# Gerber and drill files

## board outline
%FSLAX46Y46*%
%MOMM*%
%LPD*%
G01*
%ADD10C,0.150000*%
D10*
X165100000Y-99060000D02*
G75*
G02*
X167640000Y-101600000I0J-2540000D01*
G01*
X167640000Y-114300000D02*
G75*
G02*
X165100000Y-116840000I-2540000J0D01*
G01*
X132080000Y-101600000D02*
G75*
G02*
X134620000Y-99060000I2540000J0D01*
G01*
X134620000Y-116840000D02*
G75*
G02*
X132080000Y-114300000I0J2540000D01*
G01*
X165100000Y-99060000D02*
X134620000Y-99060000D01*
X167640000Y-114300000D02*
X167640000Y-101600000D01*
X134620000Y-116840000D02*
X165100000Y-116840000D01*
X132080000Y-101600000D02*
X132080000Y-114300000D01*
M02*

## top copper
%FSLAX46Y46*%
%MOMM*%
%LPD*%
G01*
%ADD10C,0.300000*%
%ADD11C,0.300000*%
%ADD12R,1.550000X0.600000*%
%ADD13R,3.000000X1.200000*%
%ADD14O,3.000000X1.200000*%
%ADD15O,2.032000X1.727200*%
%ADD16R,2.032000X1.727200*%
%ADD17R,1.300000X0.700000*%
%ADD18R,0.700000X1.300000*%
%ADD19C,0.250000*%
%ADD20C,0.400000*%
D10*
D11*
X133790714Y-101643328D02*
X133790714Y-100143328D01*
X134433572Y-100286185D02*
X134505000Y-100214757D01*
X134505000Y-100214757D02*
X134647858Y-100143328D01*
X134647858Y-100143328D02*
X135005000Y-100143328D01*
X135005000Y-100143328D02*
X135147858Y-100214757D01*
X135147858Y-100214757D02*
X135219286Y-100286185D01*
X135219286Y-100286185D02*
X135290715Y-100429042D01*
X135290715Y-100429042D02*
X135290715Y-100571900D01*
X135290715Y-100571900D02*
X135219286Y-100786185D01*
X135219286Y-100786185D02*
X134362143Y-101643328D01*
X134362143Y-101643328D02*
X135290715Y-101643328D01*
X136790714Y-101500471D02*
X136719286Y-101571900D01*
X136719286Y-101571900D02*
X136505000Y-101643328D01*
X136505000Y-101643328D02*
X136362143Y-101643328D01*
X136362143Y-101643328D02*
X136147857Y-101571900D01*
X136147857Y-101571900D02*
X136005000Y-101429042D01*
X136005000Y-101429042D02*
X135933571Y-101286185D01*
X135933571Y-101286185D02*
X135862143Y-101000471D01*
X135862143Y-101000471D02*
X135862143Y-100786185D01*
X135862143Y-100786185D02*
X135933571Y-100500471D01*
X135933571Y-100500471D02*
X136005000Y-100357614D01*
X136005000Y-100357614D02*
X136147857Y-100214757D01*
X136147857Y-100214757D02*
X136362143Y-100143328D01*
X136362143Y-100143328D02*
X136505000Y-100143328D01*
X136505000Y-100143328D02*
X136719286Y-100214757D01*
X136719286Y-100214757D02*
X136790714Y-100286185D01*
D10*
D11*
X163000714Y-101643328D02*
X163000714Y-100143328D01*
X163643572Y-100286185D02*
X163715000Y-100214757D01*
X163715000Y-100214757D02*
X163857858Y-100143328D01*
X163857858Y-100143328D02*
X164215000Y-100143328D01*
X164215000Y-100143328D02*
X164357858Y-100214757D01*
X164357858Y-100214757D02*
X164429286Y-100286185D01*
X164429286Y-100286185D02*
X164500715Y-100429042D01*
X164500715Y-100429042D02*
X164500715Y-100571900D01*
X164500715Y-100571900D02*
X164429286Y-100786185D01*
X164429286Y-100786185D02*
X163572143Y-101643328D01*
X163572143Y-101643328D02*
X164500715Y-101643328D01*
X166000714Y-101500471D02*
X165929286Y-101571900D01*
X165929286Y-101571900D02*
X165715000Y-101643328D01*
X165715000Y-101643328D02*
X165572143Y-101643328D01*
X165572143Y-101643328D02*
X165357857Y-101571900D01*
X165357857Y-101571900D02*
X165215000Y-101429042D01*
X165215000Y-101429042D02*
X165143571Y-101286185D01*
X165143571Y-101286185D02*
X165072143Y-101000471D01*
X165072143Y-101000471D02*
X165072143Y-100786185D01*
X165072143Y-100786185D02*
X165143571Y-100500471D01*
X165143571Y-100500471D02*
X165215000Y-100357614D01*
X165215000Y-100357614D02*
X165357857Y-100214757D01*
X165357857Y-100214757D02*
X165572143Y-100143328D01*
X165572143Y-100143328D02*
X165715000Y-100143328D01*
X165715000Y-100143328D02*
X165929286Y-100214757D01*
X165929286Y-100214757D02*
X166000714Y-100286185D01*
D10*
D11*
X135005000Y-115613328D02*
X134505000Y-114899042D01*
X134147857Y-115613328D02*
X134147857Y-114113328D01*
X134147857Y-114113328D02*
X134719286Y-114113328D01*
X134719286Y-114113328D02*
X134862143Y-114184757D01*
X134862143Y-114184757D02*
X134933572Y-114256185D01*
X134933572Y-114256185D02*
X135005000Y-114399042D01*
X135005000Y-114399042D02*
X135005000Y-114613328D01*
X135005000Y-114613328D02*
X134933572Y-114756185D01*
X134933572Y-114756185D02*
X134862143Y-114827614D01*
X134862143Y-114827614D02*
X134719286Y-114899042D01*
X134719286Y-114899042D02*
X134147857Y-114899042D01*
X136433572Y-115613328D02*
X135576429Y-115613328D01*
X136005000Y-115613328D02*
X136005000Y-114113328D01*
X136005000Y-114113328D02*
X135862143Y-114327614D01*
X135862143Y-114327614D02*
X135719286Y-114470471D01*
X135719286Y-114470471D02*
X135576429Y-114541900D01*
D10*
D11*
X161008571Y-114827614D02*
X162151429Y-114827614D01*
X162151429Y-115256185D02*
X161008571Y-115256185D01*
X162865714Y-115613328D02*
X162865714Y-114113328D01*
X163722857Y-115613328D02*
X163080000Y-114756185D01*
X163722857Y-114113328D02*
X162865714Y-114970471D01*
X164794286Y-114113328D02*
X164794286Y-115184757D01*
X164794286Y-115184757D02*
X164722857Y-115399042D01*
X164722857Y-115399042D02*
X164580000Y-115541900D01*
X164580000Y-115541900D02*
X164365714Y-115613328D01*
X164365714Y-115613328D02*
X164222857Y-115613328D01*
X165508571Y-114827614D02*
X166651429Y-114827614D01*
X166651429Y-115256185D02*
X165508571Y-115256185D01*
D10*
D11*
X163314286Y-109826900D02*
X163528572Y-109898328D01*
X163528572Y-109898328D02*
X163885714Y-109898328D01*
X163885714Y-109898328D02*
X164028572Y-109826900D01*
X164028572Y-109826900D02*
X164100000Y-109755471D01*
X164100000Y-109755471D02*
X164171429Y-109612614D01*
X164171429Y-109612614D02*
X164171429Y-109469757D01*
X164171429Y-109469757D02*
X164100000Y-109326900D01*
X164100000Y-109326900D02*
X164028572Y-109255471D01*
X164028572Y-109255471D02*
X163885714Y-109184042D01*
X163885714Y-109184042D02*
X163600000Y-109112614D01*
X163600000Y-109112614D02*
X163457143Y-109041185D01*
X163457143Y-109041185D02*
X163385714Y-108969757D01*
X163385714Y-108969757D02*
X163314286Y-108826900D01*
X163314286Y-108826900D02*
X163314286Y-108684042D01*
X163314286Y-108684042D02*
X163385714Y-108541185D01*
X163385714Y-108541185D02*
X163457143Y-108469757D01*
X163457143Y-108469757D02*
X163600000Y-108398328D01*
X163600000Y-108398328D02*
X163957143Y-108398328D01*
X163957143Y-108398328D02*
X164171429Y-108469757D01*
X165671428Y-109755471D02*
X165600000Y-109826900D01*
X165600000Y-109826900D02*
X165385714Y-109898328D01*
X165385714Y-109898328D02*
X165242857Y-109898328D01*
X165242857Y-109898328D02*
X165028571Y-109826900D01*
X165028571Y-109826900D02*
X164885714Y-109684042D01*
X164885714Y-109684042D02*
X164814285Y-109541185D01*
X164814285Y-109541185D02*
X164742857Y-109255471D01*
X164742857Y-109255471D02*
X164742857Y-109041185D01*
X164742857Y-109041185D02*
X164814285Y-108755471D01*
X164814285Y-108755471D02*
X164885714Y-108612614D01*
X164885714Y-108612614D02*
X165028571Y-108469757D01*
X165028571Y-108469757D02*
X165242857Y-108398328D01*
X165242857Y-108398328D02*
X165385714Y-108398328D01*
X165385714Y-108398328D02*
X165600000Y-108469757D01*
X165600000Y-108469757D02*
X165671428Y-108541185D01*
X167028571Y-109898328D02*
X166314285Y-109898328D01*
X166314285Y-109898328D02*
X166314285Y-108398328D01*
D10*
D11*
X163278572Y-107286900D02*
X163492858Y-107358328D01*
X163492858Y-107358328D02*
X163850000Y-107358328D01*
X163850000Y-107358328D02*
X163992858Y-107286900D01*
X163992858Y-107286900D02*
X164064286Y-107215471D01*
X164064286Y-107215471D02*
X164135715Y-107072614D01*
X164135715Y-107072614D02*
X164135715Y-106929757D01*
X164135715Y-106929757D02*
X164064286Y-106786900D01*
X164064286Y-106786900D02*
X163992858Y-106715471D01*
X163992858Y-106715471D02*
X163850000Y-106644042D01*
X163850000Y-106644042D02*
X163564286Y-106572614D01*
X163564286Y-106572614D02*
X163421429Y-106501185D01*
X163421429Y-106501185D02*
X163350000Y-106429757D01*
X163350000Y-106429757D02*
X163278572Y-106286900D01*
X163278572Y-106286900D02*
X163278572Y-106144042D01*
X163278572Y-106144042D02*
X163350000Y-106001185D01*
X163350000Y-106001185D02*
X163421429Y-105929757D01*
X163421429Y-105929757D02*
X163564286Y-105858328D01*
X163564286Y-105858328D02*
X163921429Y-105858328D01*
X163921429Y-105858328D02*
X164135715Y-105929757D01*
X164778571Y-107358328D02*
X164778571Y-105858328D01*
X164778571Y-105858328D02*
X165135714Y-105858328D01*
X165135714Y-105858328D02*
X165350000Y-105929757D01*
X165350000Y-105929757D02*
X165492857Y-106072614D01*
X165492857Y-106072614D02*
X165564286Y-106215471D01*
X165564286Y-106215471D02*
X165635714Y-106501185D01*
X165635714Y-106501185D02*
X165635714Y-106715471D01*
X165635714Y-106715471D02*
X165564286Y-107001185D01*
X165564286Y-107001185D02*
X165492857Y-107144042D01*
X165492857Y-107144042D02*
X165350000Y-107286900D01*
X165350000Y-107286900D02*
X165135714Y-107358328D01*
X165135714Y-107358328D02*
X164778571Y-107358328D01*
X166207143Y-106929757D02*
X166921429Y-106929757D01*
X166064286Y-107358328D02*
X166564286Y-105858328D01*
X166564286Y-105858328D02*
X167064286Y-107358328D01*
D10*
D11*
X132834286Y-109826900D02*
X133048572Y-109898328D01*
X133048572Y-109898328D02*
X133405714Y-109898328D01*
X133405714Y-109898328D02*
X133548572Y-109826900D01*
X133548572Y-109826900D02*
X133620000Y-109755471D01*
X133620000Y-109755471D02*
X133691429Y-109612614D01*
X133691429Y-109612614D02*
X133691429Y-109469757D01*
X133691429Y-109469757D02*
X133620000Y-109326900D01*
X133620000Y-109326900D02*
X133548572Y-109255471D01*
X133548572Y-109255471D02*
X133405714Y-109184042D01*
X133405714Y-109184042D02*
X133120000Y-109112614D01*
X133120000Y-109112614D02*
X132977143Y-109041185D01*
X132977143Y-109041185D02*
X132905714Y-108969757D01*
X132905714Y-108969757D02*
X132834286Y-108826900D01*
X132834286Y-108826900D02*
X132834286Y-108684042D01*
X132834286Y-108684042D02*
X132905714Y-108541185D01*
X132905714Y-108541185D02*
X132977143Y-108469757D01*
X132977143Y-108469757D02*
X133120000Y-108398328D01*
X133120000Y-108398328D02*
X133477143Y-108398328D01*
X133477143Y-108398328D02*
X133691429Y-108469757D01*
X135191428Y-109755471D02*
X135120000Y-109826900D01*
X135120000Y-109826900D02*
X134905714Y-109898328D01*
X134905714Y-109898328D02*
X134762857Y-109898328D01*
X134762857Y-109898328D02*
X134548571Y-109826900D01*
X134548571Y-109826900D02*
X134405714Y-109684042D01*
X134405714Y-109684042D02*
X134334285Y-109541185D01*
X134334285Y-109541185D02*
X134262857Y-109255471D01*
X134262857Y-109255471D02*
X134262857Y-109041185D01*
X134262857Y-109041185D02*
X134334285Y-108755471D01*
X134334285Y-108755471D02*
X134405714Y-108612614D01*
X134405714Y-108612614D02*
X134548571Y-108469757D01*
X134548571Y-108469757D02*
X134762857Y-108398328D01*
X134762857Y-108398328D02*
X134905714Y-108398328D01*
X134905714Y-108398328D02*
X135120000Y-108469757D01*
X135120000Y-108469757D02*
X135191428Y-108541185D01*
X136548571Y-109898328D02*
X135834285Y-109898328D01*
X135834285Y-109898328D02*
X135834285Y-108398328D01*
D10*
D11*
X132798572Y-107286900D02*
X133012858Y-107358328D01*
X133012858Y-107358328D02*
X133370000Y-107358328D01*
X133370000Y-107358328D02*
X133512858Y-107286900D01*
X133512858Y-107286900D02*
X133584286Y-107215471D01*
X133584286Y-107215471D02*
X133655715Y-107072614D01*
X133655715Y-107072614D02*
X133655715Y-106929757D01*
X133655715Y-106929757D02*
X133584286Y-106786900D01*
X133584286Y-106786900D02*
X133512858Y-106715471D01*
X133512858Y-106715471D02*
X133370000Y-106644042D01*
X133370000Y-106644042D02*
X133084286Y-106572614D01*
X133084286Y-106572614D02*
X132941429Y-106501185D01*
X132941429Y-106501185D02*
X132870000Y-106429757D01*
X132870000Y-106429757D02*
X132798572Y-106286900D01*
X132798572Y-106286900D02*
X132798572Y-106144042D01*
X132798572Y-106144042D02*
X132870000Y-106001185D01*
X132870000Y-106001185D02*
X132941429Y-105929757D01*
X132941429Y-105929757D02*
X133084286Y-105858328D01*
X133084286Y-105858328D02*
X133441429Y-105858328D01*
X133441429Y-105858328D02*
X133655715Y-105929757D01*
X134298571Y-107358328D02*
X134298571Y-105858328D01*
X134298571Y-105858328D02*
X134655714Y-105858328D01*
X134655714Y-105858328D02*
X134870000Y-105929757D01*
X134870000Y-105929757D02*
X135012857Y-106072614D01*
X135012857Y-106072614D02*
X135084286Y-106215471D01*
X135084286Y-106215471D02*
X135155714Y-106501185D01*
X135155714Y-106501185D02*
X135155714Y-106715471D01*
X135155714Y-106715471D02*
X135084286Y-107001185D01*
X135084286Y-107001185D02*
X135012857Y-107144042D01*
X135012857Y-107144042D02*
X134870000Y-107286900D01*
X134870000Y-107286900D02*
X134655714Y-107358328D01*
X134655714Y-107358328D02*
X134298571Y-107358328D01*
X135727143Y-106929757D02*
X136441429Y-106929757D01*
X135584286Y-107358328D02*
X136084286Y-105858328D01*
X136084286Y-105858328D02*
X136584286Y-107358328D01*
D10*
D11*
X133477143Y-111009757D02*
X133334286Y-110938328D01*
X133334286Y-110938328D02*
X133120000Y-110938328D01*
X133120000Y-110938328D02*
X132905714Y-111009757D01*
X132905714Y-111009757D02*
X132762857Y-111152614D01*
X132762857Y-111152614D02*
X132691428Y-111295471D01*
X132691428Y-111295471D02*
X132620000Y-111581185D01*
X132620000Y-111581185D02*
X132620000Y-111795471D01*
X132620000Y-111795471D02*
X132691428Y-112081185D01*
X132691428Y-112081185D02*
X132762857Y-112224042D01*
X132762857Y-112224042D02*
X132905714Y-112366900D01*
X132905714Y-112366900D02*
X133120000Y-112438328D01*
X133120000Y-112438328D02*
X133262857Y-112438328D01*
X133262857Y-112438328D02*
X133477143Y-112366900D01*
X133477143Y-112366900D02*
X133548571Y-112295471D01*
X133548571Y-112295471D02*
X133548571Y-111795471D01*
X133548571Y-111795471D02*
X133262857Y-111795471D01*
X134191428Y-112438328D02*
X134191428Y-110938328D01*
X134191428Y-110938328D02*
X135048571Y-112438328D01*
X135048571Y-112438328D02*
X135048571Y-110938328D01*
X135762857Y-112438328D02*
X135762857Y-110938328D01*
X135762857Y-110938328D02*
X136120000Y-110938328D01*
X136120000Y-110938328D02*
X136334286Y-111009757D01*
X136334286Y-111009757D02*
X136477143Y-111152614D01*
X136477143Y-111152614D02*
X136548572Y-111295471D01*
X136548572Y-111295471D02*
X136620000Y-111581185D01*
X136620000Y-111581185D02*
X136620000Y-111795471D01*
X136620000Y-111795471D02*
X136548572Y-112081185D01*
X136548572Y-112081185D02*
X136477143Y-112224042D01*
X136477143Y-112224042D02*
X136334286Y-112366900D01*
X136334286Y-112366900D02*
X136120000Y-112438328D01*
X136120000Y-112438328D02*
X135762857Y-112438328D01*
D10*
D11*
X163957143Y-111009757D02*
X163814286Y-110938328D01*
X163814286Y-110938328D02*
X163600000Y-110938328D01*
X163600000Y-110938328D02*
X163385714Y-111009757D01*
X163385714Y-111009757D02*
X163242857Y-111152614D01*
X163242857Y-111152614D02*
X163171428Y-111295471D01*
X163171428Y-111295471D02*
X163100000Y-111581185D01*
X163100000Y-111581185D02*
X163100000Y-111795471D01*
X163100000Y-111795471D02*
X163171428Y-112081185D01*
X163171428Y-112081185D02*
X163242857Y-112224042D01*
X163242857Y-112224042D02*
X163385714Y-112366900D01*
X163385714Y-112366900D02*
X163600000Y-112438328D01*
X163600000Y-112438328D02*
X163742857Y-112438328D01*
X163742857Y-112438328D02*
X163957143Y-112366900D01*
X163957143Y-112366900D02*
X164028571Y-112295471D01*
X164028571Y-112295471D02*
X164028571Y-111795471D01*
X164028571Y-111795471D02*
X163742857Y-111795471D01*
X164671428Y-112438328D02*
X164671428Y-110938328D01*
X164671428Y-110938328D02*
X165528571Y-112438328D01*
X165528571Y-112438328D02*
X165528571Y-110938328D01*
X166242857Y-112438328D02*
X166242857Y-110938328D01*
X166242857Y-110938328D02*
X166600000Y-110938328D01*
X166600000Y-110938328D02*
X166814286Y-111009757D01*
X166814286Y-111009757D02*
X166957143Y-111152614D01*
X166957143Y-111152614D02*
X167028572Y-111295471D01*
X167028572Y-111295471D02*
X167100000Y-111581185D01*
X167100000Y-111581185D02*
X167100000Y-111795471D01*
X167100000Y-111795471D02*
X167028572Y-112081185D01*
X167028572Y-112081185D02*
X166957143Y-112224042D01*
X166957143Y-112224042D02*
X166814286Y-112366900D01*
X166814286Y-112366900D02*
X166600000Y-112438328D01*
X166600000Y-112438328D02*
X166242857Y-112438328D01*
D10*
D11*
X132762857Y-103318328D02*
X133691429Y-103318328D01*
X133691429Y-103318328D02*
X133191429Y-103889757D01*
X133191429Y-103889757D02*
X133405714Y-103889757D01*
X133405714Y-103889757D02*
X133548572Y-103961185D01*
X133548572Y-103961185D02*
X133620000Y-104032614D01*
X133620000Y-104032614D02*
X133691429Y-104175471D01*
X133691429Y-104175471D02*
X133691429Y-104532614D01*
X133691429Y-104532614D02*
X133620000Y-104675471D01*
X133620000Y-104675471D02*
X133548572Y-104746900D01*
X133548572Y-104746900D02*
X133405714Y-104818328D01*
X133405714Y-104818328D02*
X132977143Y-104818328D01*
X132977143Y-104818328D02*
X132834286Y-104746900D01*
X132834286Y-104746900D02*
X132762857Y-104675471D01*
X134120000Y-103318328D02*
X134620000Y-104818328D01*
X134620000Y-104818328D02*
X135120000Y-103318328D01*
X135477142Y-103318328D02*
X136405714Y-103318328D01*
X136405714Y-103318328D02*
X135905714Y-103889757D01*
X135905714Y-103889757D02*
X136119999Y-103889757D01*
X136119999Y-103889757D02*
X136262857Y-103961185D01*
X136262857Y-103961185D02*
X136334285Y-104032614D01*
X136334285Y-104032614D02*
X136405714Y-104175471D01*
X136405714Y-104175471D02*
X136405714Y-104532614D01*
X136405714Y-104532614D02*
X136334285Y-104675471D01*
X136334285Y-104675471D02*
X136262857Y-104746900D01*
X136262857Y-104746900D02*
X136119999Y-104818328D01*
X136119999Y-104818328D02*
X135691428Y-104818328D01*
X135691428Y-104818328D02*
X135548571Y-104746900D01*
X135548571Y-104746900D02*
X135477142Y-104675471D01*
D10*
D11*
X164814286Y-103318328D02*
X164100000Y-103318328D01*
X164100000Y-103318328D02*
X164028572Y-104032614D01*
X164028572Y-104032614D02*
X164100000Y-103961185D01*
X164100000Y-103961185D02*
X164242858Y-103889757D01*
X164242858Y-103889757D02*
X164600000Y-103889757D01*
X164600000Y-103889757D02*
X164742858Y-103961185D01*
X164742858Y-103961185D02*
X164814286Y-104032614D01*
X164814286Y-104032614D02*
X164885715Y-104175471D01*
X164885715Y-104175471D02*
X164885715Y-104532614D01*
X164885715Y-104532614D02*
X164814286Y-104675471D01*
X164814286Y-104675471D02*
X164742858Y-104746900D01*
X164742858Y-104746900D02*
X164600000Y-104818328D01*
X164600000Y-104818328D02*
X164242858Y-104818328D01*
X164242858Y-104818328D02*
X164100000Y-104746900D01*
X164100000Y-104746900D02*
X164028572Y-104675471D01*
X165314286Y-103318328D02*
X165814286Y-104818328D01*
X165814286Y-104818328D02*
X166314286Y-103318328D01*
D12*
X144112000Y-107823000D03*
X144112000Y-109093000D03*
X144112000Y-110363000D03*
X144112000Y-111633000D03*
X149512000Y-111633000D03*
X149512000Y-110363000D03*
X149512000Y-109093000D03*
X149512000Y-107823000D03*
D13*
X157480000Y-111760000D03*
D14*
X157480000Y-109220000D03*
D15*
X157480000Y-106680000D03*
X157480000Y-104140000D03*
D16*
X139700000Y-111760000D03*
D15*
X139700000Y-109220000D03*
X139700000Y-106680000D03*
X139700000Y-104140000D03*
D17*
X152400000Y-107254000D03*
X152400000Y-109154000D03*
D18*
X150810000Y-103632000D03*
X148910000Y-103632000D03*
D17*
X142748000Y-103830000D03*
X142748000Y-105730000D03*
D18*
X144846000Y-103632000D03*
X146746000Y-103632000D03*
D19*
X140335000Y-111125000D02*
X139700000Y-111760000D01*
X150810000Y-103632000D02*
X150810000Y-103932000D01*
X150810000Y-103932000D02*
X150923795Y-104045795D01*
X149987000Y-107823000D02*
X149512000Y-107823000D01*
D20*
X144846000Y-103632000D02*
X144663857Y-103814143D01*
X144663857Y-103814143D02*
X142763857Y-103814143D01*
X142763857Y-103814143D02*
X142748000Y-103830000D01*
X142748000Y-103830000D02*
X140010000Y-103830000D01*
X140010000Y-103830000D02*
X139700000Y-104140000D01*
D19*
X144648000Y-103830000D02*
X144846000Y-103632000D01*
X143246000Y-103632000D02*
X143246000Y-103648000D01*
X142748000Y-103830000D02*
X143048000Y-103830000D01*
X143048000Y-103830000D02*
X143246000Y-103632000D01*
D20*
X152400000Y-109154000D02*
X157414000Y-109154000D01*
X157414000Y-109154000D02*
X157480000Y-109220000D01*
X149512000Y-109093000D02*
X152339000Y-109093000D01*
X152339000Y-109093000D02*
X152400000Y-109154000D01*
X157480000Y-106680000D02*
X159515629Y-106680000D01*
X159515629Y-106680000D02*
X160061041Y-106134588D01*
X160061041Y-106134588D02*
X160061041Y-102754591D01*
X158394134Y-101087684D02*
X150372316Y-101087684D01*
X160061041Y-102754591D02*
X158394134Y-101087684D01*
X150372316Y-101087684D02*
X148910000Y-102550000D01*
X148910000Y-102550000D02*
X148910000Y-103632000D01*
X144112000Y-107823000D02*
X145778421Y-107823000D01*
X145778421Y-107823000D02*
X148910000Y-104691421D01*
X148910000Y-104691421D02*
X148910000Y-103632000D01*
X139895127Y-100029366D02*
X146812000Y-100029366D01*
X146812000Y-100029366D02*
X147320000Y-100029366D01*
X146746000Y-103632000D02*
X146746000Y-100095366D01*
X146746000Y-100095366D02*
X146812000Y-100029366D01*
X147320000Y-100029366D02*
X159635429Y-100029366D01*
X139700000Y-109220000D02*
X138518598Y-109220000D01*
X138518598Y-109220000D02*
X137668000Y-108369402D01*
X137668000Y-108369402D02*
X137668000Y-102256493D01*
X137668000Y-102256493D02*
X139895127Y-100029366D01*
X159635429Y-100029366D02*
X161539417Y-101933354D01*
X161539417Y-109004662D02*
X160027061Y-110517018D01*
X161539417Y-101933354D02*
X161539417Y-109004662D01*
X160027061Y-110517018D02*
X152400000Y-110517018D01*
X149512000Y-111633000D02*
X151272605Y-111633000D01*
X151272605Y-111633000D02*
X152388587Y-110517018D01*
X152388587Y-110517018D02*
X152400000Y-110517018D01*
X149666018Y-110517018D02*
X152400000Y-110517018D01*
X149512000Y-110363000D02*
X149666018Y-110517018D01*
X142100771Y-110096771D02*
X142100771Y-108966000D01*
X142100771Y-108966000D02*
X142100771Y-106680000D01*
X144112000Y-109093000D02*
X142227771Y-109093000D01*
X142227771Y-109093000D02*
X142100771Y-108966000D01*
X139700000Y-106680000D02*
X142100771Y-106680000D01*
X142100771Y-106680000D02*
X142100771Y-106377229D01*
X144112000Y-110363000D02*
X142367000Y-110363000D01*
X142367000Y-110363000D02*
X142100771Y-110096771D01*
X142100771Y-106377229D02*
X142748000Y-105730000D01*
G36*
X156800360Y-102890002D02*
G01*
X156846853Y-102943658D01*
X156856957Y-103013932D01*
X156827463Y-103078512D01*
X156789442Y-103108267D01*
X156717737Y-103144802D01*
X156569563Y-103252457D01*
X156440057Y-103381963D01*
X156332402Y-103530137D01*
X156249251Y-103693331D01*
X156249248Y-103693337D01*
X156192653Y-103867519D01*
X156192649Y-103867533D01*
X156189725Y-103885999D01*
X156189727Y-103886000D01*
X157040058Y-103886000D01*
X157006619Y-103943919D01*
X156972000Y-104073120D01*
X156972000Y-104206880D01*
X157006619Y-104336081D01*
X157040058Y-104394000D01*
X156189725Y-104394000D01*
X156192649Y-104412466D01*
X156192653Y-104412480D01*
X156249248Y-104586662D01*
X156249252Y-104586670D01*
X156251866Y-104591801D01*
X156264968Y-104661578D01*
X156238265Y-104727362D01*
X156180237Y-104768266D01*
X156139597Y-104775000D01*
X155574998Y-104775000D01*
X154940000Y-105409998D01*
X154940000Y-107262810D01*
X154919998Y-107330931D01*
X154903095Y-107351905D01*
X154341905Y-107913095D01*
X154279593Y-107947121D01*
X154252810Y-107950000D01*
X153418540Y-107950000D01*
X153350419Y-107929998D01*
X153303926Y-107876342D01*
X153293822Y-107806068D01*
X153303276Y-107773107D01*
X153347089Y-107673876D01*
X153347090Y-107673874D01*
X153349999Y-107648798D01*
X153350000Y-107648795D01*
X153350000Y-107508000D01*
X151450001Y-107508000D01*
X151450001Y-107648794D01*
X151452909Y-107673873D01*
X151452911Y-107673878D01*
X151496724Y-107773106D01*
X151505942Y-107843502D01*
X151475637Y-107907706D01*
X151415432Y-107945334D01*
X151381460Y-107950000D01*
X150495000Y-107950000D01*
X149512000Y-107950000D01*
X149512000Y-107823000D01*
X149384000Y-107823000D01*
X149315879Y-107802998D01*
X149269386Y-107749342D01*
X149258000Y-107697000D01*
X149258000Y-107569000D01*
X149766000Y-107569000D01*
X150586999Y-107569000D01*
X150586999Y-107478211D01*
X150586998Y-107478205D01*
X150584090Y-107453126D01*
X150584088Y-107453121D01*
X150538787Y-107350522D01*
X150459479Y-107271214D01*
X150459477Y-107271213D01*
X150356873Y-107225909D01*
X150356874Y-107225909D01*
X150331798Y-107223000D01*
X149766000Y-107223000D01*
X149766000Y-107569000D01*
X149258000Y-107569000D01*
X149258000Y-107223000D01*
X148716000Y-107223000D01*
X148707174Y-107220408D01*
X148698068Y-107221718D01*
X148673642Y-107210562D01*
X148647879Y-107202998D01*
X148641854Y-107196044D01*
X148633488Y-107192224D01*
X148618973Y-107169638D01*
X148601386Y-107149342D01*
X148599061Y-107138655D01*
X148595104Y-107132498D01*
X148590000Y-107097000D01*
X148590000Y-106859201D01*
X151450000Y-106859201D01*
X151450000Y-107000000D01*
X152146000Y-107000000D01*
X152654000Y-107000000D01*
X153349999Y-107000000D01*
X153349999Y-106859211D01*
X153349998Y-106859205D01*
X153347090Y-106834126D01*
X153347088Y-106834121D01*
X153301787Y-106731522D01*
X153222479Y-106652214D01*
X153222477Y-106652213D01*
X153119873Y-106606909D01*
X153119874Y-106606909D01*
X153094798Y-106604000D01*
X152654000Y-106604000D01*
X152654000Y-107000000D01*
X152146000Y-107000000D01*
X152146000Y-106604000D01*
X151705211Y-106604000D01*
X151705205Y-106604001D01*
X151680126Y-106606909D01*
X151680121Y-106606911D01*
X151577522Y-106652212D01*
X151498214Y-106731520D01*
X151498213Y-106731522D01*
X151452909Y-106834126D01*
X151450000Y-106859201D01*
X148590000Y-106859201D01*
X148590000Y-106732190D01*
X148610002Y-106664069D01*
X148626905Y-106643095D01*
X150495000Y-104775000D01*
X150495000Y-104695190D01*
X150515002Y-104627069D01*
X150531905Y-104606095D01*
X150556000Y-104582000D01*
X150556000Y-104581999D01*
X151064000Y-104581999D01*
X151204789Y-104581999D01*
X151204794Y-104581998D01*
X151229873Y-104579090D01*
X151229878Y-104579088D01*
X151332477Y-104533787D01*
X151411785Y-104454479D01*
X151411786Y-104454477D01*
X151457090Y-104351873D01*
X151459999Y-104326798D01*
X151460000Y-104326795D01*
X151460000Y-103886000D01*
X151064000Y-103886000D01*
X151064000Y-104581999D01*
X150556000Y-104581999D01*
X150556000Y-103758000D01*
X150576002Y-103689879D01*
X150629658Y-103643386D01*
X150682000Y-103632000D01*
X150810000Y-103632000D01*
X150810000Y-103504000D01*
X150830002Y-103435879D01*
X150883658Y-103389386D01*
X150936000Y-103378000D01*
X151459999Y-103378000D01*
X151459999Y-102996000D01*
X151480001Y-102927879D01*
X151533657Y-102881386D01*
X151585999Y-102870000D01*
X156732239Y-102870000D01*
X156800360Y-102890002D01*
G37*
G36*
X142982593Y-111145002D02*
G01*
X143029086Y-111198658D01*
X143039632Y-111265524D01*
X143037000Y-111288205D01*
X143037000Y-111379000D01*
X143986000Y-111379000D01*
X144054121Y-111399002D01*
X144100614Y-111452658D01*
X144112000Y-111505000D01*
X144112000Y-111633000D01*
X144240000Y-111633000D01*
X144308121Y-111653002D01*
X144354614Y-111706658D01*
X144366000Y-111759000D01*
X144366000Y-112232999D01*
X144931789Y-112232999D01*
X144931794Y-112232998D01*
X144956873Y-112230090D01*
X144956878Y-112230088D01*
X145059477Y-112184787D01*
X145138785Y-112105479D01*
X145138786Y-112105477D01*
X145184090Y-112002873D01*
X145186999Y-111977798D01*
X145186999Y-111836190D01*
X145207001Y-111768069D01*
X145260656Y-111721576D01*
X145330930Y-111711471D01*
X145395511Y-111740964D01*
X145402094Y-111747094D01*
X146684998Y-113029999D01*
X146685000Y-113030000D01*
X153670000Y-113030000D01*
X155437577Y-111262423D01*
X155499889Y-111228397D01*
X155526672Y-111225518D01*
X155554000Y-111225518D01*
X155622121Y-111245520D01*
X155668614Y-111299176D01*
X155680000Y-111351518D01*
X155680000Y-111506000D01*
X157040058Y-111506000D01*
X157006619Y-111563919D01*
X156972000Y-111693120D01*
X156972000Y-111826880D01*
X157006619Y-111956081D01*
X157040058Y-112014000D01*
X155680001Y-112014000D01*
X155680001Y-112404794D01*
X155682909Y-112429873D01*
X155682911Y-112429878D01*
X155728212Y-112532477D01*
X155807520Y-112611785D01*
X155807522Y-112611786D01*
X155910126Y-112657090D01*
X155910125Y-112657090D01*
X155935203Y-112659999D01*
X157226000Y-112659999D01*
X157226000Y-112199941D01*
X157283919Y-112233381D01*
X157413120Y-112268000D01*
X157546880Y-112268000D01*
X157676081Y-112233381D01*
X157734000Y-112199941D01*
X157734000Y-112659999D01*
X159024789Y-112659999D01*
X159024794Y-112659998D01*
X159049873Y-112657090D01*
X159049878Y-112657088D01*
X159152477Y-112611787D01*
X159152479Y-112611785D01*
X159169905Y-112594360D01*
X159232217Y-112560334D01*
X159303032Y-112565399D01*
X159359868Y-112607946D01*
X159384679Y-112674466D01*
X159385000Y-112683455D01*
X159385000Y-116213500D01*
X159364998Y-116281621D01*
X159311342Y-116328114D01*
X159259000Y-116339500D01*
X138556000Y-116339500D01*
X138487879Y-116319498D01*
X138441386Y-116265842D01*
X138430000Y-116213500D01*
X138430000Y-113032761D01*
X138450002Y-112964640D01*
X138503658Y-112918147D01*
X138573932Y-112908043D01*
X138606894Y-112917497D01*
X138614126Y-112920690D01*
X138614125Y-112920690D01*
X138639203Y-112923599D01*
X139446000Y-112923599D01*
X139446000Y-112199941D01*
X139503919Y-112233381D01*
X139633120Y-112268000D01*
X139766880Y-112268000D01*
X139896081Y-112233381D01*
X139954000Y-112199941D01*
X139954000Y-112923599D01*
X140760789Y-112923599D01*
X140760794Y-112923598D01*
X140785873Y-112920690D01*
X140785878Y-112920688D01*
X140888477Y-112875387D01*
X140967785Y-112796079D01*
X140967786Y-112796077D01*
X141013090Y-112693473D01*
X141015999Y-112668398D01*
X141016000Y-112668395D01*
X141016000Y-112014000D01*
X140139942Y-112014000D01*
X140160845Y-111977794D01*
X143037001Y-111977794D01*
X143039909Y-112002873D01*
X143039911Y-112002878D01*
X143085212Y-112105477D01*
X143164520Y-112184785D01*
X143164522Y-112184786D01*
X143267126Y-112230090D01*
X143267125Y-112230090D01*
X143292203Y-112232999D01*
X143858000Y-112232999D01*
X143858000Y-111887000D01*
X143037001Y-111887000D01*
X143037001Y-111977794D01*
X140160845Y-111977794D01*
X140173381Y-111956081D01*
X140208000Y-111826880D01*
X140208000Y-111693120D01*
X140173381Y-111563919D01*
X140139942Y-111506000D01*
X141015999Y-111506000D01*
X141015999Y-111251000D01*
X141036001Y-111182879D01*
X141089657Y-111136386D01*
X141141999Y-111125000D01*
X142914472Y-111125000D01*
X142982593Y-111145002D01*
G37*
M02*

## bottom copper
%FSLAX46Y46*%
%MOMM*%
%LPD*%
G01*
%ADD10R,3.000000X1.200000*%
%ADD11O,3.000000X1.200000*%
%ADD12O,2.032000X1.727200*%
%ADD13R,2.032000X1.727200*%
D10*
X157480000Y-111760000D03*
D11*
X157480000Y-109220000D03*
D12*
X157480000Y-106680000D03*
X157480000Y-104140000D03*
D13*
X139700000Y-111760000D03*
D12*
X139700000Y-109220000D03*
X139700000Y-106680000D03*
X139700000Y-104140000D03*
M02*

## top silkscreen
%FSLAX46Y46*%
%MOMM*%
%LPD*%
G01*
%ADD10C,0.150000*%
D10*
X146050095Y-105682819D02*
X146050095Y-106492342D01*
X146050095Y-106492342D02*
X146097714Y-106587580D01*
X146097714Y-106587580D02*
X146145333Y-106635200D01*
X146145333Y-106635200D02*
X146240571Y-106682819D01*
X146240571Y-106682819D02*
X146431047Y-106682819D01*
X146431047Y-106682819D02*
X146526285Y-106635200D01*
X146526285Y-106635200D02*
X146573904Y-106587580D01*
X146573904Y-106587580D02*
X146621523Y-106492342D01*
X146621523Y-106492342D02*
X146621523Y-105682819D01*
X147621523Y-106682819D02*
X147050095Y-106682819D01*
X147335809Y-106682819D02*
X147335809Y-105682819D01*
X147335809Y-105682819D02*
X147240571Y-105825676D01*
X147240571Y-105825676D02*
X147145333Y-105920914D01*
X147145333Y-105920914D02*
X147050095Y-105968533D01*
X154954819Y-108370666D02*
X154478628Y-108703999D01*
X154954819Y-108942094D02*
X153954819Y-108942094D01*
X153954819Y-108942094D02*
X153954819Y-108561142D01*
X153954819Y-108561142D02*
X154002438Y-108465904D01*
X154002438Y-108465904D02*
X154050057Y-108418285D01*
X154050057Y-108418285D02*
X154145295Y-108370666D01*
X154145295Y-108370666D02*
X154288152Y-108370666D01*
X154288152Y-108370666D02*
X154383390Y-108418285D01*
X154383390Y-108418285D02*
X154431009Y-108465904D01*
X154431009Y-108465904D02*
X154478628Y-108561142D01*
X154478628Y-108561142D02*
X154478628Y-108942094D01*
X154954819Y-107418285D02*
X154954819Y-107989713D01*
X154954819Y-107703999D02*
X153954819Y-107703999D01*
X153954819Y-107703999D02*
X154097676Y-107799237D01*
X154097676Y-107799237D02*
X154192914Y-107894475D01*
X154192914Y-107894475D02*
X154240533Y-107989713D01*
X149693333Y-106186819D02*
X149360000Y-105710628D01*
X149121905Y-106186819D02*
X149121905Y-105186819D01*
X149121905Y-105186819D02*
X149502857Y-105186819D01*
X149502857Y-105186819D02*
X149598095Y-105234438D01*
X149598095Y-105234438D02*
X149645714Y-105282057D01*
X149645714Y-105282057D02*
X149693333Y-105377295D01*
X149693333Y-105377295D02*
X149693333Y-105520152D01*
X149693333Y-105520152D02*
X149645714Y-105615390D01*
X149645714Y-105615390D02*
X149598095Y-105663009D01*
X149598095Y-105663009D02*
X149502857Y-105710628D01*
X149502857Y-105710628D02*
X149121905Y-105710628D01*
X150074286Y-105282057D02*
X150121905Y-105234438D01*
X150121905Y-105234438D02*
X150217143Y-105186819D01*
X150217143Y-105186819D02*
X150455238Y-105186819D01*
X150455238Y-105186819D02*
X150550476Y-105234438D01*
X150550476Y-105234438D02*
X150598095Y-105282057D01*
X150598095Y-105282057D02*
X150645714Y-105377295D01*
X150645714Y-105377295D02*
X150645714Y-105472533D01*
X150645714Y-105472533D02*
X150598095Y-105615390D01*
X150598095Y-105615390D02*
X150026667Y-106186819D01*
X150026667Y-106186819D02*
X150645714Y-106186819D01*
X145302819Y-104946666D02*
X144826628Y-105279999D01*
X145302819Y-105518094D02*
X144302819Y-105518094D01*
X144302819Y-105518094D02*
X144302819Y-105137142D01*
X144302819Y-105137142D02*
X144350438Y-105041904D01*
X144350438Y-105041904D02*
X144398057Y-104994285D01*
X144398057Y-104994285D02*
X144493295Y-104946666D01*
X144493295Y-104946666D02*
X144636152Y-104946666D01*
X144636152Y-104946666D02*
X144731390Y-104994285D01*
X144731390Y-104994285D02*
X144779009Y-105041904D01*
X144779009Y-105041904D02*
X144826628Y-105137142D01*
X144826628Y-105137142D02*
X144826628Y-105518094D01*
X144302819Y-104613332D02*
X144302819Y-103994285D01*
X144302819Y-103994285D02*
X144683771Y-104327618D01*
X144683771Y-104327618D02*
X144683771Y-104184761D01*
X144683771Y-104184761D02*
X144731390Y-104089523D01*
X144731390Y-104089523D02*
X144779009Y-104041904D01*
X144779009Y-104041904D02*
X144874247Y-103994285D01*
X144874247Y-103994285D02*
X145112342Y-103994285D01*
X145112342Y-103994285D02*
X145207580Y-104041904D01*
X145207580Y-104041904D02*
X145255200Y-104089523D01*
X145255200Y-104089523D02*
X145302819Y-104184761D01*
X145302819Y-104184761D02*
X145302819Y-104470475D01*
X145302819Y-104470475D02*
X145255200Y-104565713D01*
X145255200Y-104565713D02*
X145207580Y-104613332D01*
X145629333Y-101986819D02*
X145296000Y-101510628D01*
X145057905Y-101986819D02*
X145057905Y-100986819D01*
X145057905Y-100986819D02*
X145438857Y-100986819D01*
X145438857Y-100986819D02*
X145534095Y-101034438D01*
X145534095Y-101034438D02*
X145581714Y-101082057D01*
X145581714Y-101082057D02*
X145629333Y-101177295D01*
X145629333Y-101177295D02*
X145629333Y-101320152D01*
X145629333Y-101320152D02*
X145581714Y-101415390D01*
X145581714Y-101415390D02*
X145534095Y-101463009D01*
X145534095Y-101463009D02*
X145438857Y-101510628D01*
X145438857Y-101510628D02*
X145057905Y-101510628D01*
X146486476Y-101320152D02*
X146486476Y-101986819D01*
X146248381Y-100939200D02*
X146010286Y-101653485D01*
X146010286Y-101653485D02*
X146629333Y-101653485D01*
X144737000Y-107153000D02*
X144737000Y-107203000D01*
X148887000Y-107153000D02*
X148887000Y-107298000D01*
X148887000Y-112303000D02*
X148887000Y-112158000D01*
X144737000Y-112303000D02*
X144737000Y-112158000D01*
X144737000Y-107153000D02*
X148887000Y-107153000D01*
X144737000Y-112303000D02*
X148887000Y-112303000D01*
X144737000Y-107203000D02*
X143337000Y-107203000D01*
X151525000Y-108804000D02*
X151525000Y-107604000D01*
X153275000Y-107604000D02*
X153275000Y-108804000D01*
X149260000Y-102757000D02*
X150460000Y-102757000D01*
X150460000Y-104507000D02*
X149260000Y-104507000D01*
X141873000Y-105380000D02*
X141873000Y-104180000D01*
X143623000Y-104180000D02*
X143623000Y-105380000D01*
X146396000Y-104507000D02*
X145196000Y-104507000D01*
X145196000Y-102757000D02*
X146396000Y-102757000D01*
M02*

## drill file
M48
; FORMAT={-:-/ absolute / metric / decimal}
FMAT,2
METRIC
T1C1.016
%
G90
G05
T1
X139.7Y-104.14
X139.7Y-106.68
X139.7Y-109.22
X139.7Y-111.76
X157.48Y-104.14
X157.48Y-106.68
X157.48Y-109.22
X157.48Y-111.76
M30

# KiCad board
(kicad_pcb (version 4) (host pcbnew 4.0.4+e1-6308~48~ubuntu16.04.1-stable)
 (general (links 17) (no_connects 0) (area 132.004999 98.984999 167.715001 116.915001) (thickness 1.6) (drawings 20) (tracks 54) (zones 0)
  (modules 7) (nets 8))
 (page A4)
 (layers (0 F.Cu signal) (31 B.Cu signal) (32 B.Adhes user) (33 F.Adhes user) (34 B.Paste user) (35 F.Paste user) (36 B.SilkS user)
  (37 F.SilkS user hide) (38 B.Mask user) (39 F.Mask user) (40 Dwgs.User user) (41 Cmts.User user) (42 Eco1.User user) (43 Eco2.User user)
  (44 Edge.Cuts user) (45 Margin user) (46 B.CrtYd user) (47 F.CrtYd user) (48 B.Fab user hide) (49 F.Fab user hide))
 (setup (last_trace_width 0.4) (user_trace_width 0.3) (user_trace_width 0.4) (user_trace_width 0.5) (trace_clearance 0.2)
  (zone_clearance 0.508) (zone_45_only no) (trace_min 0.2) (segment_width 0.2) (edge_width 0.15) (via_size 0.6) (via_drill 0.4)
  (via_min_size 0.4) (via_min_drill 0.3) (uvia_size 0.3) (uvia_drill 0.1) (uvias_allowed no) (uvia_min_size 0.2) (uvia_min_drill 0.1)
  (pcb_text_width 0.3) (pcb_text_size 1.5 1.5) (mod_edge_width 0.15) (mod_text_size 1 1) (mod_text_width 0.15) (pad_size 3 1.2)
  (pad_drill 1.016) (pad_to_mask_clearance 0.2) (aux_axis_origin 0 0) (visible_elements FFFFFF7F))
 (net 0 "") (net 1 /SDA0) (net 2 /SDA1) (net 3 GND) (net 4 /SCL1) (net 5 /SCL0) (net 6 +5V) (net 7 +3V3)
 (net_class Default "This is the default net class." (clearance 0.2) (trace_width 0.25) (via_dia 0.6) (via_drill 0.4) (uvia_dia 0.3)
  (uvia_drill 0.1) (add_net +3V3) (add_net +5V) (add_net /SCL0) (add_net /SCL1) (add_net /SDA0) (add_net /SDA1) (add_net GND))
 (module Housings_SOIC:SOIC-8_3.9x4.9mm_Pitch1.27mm (layer F.Cu) (at 146.812 109.728)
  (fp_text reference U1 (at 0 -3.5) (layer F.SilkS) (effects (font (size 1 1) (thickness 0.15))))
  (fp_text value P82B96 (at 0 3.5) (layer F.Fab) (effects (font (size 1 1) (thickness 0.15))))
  (fp_line (start -2.075 -2.575) (end -2.075 -2.525) (layer F.SilkS) (width 0.15))
  (fp_line (start 2.075 -2.575) (end 2.075 -2.43) (layer F.SilkS) (width 0.15))
  (fp_line (start 2.075 2.575) (end 2.075 2.43) (layer F.SilkS) (width 0.15))
  (fp_line (start -2.075 2.575) (end -2.075 2.43) (layer F.SilkS) (width 0.15))
  (fp_line (start -2.075 -2.575) (end 2.075 -2.575) (layer F.SilkS) (width 0.15))
  (fp_line (start -2.075 2.575) (end 2.075 2.575) (layer F.SilkS) (width 0.15))
  (fp_line (start -2.075 -2.525) (end -3.475 -2.525) (layer F.SilkS) (width 0.15))
  (pad 1 smd rect (at -2.7 -1.905) (size 1.55 0.6) (layers F.Cu F.Paste F.Mask) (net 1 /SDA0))
  (pad 2 smd rect (at -2.7 -0.635) (size 1.55 0.6) (layers F.Cu F.Paste F.Mask) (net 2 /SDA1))
  (pad 3 smd rect (at -2.7 0.635) (size 1.55 0.6) (layers F.Cu F.Paste F.Mask) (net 2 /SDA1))
  (pad 4 smd rect (at -2.7 1.905) (size 1.55 0.6) (layers F.Cu F.Paste F.Mask) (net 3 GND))
  (pad 5 smd rect (at 2.7 1.905) (size 1.55 0.6) (layers F.Cu F.Paste F.Mask) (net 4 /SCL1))
  (pad 6 smd rect (at 2.7 0.635) (size 1.55 0.6) (layers F.Cu F.Paste F.Mask) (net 4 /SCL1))
  (pad 7 smd rect (at 2.7 -0.635) (size 1.55 0.6) (layers F.Cu F.Paste F.Mask) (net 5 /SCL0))
  (pad 8 smd rect (at 2.7 -1.905) (size 1.55 0.6) (layers F.Cu F.Paste F.Mask) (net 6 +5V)))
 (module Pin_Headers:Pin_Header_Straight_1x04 (layer B.Cu) (at 157.48 111.76)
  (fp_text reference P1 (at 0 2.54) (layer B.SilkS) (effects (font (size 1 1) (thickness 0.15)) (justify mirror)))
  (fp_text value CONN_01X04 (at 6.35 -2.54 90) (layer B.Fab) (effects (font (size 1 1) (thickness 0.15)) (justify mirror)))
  (pad 1 thru_hole rect (at 0 0) (size 3 1.2) (drill 1.016) (layers *.Cu *.Mask B.SilkS) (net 3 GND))
  (pad 2 thru_hole oval (at 0 -2.54) (size 3 1.2) (drill 1.016) (layers *.Cu *.Mask B.SilkS) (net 5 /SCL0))
  (pad 3 thru_hole oval (at 0 -5.08) (size 2.032 1.7272) (drill 1.016) (layers *.Cu *.Mask B.SilkS) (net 1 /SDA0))
  (pad 4 thru_hole oval (at 0 -7.62) (size 2.032 1.7272) (drill 1.016) (layers *.Cu *.Mask B.SilkS) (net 6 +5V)))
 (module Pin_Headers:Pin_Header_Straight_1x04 (layer B.Cu) (at 139.7 111.76)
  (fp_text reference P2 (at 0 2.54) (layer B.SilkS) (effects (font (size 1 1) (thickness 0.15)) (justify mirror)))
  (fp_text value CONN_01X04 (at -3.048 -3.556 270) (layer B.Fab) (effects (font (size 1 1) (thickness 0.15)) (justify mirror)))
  (pad 1 thru_hole rect (at 0 0) (size 2.032 1.7272) (drill 1.016) (layers *.Cu *.Mask B.SilkS) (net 3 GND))
  (pad 2 thru_hole oval (at 0 -2.54) (size 2.032 1.7272) (drill 1.016) (layers *.Cu *.Mask B.SilkS) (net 4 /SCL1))
  (pad 3 thru_hole oval (at 0 -5.08) (size 2.032 1.7272) (drill 1.016) (layers *.Cu *.Mask B.SilkS) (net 2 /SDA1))
  (pad 4 thru_hole oval (at 0 -7.62) (size 2.032 1.7272) (drill 1.016) (layers *.Cu *.Mask B.SilkS) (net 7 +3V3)))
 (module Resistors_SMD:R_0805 (layer F.Cu) (at 152.4 108.204 270)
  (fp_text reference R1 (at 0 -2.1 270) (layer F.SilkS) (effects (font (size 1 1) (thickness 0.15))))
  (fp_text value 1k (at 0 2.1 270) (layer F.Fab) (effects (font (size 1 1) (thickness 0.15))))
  (fp_line (start 0.6 0.875) (end -0.6 0.875) (layer F.SilkS) (width 0.15))
  (fp_line (start -0.6 -0.875) (end 0.6 -0.875) (layer F.SilkS) (width 0.15))
  (pad 1 smd rect (at -0.95 0 270) (size 0.7 1.3) (layers F.Cu F.Paste F.Mask) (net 6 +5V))
  (pad 2 smd rect (at 0.95 0 270) (size 0.7 1.3) (layers F.Cu F.Paste F.Mask) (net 5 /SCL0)))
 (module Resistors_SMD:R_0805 (layer F.Cu) (at 149.86 103.632 180)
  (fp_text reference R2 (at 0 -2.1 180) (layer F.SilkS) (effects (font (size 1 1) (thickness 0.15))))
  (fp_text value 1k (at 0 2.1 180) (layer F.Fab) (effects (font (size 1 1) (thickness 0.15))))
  (fp_line (start 0.6 0.875) (end -0.6 0.875) (layer F.SilkS) (width 0.15))
  (fp_line (start -0.6 -0.875) (end 0.6 -0.875) (layer F.SilkS) (width 0.15))
  (pad 1 smd rect (at -0.95 0 180) (size 0.7 1.3) (layers F.Cu F.Paste F.Mask) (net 6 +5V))
  (pad 2 smd rect (at 0.95 0 180) (size 0.7 1.3) (layers F.Cu F.Paste F.Mask) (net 1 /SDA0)))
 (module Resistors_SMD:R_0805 (layer F.Cu) (at 142.748 104.78 270)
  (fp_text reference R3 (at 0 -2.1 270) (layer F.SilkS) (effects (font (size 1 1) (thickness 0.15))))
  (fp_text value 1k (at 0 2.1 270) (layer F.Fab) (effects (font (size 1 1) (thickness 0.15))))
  (fp_line (start 0.6 0.875) (end -0.6 0.875) (layer F.SilkS) (width 0.15))
  (fp_line (start -0.6 -0.875) (end 0.6 -0.875) (layer F.SilkS) (width 0.15))
  (pad 1 smd rect (at -0.95 0 270) (size 0.7 1.3) (layers F.Cu F.Paste F.Mask) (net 7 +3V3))
  (pad 2 smd rect (at 0.95 0 270) (size 0.7 1.3) (layers F.Cu F.Paste F.Mask) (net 2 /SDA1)))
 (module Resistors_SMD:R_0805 (layer F.Cu) (at 145.796 103.632)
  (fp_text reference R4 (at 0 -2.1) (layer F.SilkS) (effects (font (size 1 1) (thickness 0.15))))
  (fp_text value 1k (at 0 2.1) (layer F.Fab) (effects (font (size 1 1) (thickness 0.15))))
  (fp_line (start 0.6 0.875) (end -0.6 0.875) (layer F.SilkS) (width 0.15))
  (fp_line (start -0.6 -0.875) (end 0.6 -0.875) (layer F.SilkS) (width 0.15))
  (pad 1 smd rect (at -0.95 0) (size 0.7 1.3) (layers F.Cu F.Paste F.Mask) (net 7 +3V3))
  (pad 2 smd rect (at 0.95 0) (size 0.7 1.3) (layers F.Cu F.Paste F.Mask) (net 4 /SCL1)))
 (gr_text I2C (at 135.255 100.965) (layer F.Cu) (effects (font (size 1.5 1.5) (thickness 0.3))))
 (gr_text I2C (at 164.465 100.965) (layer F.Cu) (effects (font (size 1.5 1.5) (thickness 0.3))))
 (gr_arc (start 165.1 101.6) (end 165.1 99.06) (angle 90) (layer Edge.Cuts) (width 0.15))
 (gr_arc (start 165.1 114.3) (end 167.64 114.3) (angle 90) (layer Edge.Cuts) (width 0.15))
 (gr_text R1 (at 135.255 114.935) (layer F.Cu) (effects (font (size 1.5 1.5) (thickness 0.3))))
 (gr_arc (start 134.62 101.6) (end 132.08 101.6) (angle 90) (layer Edge.Cuts) (width 0.15))
 (gr_arc (start 134.62 114.3) (end 134.62 116.84) (angle 90) (layer Edge.Cuts) (width 0.15))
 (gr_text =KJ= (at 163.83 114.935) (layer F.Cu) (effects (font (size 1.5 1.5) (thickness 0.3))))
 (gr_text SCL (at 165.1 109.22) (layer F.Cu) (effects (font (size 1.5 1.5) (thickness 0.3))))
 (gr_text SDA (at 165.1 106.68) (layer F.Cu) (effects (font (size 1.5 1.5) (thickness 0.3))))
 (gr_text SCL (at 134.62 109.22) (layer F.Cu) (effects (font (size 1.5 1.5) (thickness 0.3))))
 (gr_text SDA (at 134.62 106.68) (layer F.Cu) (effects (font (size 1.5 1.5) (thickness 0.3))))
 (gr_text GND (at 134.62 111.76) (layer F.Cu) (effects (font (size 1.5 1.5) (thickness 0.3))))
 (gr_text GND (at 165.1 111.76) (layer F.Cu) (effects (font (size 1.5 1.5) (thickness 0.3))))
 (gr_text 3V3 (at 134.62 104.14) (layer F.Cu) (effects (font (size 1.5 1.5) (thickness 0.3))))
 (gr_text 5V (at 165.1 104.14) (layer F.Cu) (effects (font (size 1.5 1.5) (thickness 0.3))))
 (gr_line (start 165.1 99.06) (end 134.62 99.06) (layer Edge.Cuts) (width 0.15))
 (gr_line (start 167.64 114.3) (end 167.64 101.6) (layer Edge.Cuts) (width 0.15))
 (gr_line (start 134.62 116.84) (end 165.1 116.84) (layer Edge.Cuts) (width 0.15))
 (gr_line (start 132.08 101.6) (end 132.08 114.3) (layer Edge.Cuts) (width 0.15))
 (segment (start 140.335 111.125) (end 139.7 111.76) (width 0.25) (layer F.Cu) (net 3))
 (segment (start 150.81 103.632) (end 150.81 103.932) (width 0.25) (layer F.Cu) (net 6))
 (segment (start 150.81 103.932) (end 150.923795 104.045795) (width 0.25) (layer F.Cu) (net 6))
 (segment (start 149.987 107.823) (end 149.512 107.823) (width 0.25) (layer F.Cu) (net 6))
 (segment (start 144.846 103.632) (end 144.663857 103.814143) (width 0.4) (layer F.Cu) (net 7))
 (segment (start 144.663857 103.814143) (end 142.763857 103.814143) (width 0.4) (layer F.Cu) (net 7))
 (segment (start 142.763857 103.814143) (end 142.748 103.83) (width 0.4) (layer F.Cu) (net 7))
 (segment (start 142.748 103.83) (end 140.01 103.83) (width 0.4) (layer F.Cu) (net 7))
 (segment (start 140.01 103.83) (end 139.7 104.14) (width 0.4) (layer F.Cu) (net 7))
 (segment (start 144.648 103.83) (end 144.846 103.632) (width 0.25) (layer F.Cu) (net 7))
 (segment (start 143.246 103.632) (end 143.246 103.648) (width 0.25) (layer F.Cu) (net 7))
 (segment (start 142.748 103.83) (end 143.048 103.83) (width 0.25) (layer F.Cu) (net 7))
 (segment (start 143.048 103.83) (end 143.246 103.632) (width 0.25) (layer F.Cu) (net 7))
 (segment (start 152.4 109.154) (end 157.414 109.154) (width 0.4) (layer F.Cu) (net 5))
 (segment (start 157.414 109.154) (end 157.48 109.22) (width 0.4) (layer F.Cu) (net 5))
 (segment (start 149.512 109.093) (end 152.339 109.093) (width 0.4) (layer F.Cu) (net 5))
 (segment (start 152.339 109.093) (end 152.4 109.154) (width 0.4) (layer F.Cu) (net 5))
 (segment (start 157.48 106.68) (end 159.515629 106.68) (width 0.4) (layer F.Cu) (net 1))
 (segment (start 159.515629 106.68) (end 160.061041 106.134588) (width 0.4) (layer F.Cu) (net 1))
 (segment (start 160.061041 106.134588) (end 160.061041 102.754591) (width 0.4) (layer F.Cu) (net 1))
 (segment (start 158.394134 101.087684) (end 150.372316 101.087684) (width 0.4) (layer F.Cu) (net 1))
 (segment (start 160.061041 102.754591) (end 158.394134 101.087684) (width 0.4) (layer F.Cu) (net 1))
 (segment (start 150.372316 101.087684) (end 148.91 102.55) (width 0.4) (layer F.Cu) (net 1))
 (segment (start 148.91 102.55) (end 148.91 103.632) (width 0.4) (layer F.Cu) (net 1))
 (segment (start 144.112 107.823) (end 145.778421 107.823) (width 0.4) (layer F.Cu) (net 1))
 (segment (start 145.778421 107.823) (end 148.91 104.691421) (width 0.4) (layer F.Cu) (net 1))
 (segment (start 148.91 104.691421) (end 148.91 103.632) (width 0.4) (layer F.Cu) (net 1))
 (segment (start 139.895127 100.029366) (end 146.812 100.029366) (width 0.4) (layer F.Cu) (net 4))
 (segment (start 146.812 100.029366) (end 147.32 100.029366) (width 0.4) (layer F.Cu) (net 4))
 (segment (start 146.746 103.632) (end 146.746 100.095366) (width 0.4) (layer F.Cu) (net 4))
 (segment (start 146.746 100.095366) (end 146.812 100.029366) (width 0.4) (layer F.Cu) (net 4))
 (segment (start 147.32 100.029366) (end 159.635429 100.029366) (width 0.4) (layer F.Cu) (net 4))
 (segment (start 139.7 109.22) (end 138.518598 109.22) (width 0.4) (layer F.Cu) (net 4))
 (segment (start 138.518598 109.22) (end 137.668 108.369402) (width 0.4) (layer F.Cu) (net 4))
 (segment (start 137.668 108.369402) (end 137.668 102.256493) (width 0.4) (layer F.Cu) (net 4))
 (segment (start 137.668 102.256493) (end 139.895127 100.029366) (width 0.4) (layer F.Cu) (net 4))
 (segment (start 159.635429 100.029366) (end 161.539417 101.933354) (width 0.4) (layer F.Cu) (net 4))
 (segment (start 161.539417 109.004662) (end 160.027061 110.517018) (width 0.4) (layer F.Cu) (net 4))
 (segment (start 161.539417 101.933354) (end 161.539417 109.004662) (width 0.4) (layer F.Cu) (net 4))
 (segment (start 160.027061 110.517018) (end 152.4 110.517018) (width 0.4) (layer F.Cu) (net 4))
 (segment (start 149.512 111.633) (end 151.272605 111.633) (width 0.4) (layer F.Cu) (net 4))
 (segment (start 151.272605 111.633) (end 152.388587 110.517018) (width 0.4) (layer F.Cu) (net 4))
 (segment (start 152.388587 110.517018) (end 152.4 110.517018) (width 0.4) (layer F.Cu) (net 4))
 (segment (start 149.666018 110.517018) (end 152.4 110.517018) (width 0.4) (layer F.Cu) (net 4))
 (segment (start 149.512 110.363) (end 149.666018 110.517018) (width 0.4) (layer F.Cu) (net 4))
 (segment (start 142.100771 110.096771) (end 142.100771 108.966) (width 0.4) (layer F.Cu) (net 2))
 (segment (start 142.100771 108.966) (end 142.100771 106.68) (width 0.4) (layer F.Cu) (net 2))
 (segment (start 144.112 109.093) (end 142.227771 109.093) (width 0.4) (layer F.Cu) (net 2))
 (segment (start 142.227771 109.093) (end 142.100771 108.966) (width 0.4) (layer F.Cu) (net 2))
 (segment (start 139.7 106.68) (end 142.100771 106.68) (width 0.4) (layer F.Cu) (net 2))
 (segment (start 142.100771 106.68) (end 142.100771 106.377229) (width 0.4) (layer F.Cu) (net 2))
 (segment (start 144.112 110.363) (end 142.367 110.363) (width 0.4) (layer F.Cu) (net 2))
 (segment (start 142.367 110.363) (end 142.100771 110.096771) (width 0.4) (layer F.Cu) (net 2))
 (segment (start 142.100771 106.377229) (end 142.748 105.73) (width 0.4) (layer F.Cu) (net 2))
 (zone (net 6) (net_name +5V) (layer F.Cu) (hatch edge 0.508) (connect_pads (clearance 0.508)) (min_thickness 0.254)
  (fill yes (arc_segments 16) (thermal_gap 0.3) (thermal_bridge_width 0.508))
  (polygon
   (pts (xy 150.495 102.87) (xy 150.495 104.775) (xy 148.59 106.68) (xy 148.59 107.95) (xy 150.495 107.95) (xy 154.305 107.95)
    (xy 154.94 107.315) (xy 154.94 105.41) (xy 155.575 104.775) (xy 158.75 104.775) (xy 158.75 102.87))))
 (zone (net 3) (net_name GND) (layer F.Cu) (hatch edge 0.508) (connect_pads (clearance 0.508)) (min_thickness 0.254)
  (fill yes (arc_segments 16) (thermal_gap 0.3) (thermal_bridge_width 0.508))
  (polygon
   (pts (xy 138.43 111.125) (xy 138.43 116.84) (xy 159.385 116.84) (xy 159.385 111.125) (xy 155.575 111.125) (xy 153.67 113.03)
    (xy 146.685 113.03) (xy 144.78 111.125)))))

